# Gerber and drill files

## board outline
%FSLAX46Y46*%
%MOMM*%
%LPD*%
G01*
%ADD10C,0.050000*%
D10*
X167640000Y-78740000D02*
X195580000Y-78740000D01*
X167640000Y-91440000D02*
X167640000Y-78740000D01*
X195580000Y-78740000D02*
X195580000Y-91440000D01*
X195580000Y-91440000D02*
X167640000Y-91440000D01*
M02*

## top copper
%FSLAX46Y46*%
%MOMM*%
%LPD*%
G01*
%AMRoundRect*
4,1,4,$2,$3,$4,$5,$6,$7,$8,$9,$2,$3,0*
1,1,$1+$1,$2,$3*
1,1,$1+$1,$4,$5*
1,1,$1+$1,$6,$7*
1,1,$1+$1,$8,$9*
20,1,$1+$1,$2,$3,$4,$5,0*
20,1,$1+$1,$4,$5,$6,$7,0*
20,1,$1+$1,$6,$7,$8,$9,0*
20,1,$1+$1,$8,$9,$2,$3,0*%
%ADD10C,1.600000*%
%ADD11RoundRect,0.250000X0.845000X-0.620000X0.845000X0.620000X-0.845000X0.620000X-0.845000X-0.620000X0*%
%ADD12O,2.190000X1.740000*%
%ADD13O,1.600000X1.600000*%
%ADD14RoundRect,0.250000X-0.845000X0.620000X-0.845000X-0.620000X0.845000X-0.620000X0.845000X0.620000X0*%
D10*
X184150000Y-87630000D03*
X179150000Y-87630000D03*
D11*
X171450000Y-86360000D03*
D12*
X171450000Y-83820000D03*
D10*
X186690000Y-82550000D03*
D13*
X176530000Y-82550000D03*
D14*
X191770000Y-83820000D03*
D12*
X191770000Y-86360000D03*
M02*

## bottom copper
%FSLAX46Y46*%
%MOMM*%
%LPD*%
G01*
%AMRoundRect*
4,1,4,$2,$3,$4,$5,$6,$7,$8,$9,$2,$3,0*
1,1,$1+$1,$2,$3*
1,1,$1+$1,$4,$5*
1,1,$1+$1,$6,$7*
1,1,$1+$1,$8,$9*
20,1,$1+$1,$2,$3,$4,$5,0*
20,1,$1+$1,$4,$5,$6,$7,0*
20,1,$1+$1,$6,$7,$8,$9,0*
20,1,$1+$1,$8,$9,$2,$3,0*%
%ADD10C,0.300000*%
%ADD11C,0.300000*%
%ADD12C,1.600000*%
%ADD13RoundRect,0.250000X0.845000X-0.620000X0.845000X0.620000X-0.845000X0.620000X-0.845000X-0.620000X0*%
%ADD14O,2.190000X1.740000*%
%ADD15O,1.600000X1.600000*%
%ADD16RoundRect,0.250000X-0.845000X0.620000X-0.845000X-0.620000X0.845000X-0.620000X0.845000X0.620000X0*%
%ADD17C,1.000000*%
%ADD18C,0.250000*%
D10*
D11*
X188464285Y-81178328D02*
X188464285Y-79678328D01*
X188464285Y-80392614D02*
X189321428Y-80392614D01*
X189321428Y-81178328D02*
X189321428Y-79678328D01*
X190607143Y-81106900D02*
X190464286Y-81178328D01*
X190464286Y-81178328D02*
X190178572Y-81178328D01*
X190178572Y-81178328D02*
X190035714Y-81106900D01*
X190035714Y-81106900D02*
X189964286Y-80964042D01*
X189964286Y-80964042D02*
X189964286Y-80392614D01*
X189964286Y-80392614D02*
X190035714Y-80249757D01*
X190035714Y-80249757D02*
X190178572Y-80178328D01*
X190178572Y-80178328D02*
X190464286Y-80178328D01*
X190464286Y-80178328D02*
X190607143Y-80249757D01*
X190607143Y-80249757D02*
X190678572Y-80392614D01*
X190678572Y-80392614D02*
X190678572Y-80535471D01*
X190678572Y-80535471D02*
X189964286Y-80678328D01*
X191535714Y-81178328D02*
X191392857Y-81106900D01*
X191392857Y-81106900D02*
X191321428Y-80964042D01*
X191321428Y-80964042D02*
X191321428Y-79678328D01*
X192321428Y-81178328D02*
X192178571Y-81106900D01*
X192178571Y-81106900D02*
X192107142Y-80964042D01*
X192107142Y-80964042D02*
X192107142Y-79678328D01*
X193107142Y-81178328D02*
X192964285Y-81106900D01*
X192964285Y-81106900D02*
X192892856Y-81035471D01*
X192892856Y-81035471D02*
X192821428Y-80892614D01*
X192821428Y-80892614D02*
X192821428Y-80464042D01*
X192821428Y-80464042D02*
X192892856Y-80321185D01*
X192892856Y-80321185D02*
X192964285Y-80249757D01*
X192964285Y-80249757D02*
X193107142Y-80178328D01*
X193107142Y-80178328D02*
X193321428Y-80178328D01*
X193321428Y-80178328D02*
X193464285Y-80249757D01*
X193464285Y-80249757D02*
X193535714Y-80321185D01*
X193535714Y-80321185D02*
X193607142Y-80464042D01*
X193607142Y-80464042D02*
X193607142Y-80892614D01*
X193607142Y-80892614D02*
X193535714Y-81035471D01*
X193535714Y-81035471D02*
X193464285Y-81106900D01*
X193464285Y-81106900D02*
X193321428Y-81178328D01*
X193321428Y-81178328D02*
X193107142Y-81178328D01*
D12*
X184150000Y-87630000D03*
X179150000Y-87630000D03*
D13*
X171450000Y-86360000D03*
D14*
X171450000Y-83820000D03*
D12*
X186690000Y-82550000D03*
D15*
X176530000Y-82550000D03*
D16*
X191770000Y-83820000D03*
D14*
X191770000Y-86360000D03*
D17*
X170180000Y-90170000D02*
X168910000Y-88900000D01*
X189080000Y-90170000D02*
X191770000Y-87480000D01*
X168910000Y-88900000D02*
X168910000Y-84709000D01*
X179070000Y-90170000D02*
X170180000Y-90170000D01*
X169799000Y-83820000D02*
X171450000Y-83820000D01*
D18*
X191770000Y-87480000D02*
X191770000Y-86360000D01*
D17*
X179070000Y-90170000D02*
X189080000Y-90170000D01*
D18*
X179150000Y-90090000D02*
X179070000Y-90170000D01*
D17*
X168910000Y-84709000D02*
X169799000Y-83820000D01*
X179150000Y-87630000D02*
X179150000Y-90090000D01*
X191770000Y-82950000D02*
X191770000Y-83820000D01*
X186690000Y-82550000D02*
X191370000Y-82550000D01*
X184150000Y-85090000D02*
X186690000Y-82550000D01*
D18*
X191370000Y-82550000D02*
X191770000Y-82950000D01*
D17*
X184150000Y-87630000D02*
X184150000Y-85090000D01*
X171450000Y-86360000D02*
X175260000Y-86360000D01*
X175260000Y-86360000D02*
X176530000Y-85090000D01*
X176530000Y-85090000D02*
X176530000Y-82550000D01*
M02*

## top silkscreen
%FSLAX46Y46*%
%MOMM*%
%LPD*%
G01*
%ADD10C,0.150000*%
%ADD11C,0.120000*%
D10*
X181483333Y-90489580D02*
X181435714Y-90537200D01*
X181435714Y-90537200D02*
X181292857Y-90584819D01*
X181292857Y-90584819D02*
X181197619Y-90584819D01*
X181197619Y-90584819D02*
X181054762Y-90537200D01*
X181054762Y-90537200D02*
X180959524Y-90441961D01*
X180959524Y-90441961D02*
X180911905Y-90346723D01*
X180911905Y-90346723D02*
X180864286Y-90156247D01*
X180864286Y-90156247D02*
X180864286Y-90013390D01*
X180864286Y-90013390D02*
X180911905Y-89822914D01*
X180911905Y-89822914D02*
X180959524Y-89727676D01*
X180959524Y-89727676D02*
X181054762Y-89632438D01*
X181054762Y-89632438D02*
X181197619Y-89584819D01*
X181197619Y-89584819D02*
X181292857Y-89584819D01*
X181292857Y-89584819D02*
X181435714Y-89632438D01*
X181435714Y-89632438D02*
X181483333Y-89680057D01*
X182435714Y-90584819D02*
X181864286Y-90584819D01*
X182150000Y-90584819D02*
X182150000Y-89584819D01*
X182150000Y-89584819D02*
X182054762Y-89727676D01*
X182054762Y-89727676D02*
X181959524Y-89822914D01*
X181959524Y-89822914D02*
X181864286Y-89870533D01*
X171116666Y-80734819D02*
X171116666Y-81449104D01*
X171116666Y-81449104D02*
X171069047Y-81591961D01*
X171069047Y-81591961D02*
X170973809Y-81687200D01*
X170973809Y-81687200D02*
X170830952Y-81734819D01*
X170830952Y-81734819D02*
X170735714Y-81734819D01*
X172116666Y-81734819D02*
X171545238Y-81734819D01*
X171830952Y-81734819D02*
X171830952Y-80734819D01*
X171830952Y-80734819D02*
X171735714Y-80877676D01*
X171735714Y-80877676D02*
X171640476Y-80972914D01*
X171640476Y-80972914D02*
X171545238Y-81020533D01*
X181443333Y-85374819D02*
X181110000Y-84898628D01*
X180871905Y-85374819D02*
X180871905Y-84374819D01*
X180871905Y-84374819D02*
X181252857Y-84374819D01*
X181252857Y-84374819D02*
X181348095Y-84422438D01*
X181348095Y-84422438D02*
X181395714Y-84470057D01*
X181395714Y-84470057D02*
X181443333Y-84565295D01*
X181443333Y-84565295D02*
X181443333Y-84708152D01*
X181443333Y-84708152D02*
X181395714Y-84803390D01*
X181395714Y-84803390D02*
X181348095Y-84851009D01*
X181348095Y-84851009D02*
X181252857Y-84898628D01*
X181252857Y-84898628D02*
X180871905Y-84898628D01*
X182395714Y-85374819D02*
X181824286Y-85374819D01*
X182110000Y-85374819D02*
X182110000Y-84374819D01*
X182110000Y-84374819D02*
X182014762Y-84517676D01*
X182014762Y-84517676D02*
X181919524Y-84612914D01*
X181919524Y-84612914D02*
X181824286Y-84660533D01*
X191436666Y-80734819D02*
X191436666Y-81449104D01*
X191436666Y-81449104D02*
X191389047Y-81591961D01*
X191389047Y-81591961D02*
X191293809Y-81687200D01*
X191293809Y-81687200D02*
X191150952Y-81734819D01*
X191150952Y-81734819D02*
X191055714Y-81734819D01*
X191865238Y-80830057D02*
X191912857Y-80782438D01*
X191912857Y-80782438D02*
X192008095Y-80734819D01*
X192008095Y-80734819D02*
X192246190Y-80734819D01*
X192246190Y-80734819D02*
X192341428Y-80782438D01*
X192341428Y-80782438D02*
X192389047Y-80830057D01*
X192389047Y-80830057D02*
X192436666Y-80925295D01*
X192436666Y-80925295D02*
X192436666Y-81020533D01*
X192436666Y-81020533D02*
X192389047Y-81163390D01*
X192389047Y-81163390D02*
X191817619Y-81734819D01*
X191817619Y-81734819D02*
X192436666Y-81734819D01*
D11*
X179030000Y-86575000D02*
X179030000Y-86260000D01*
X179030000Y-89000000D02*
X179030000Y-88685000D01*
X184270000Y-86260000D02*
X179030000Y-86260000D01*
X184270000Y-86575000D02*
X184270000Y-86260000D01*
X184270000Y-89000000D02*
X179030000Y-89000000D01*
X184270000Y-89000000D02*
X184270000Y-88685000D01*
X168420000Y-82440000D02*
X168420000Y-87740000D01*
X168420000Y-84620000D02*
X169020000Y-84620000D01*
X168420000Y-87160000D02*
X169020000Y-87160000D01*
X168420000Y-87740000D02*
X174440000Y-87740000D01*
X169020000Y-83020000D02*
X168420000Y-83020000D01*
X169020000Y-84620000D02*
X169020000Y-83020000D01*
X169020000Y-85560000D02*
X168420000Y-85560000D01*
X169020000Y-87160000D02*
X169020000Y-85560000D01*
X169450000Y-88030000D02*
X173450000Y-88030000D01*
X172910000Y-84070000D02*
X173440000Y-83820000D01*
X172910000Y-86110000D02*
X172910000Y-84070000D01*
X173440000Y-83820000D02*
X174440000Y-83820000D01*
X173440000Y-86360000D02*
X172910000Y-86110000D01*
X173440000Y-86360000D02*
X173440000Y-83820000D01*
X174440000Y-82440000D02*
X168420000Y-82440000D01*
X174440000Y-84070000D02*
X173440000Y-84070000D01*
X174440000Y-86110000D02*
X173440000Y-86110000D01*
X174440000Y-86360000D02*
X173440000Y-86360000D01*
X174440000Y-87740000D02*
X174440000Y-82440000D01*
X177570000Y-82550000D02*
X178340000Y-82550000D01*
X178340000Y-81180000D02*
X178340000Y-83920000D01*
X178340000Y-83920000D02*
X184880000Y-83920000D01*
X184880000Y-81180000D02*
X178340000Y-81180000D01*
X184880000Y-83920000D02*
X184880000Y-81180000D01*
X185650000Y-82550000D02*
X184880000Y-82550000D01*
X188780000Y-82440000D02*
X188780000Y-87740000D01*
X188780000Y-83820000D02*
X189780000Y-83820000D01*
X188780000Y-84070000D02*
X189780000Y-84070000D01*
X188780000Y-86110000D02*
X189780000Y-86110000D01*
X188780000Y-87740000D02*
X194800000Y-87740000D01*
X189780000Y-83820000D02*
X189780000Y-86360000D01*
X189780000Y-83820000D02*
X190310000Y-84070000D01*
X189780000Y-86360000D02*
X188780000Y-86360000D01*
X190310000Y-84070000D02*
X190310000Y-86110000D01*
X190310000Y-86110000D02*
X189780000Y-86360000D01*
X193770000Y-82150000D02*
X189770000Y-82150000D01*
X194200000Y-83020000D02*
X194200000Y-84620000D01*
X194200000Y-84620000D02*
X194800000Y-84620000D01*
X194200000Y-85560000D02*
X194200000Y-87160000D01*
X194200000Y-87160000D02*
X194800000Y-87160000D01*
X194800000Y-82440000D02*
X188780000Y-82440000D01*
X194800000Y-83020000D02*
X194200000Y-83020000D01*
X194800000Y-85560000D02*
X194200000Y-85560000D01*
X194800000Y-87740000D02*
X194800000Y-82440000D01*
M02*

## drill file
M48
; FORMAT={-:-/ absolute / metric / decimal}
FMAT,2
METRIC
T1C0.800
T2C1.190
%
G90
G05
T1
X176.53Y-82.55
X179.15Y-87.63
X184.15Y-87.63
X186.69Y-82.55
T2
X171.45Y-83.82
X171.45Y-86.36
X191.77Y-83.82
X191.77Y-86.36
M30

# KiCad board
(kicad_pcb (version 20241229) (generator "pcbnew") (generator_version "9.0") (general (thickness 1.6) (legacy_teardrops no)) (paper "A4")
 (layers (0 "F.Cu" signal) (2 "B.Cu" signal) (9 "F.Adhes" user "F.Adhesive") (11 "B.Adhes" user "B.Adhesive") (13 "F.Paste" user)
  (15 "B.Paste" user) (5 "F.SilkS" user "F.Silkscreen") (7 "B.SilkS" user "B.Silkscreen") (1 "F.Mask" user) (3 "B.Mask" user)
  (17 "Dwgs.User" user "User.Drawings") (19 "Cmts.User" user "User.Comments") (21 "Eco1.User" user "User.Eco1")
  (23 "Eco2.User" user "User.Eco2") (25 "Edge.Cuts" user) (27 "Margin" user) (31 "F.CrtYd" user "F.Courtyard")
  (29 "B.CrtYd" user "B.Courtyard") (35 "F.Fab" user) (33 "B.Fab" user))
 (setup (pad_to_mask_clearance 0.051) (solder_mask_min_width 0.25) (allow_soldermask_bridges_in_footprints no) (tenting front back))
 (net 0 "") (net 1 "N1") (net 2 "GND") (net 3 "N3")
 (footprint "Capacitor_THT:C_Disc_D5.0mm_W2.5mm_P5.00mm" (layer "F.Cu") (at 184.15 87.63 180)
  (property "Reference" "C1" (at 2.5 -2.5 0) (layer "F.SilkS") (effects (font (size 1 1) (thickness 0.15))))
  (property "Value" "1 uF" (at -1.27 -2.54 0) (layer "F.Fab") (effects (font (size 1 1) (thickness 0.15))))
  (fp_line (start 5.12 1.055) (end 5.12 1.37) (stroke (width 0.12) (type solid)) (layer "F.SilkS"))
  (fp_line (start 5.12 -1.37) (end 5.12 -1.055) (stroke (width 0.12) (type solid)) (layer "F.SilkS"))
  (fp_line (start -0.12 1.37) (end 5.12 1.37) (stroke (width 0.12) (type solid)) (layer "F.SilkS"))
  (fp_line (start -0.12 1.055) (end -0.12 1.37) (stroke (width 0.12) (type solid)) (layer "F.SilkS"))
  (fp_line (start -0.12 -1.37) (end 5.12 -1.37) (stroke (width 0.12) (type solid)) (layer "F.SilkS"))
  (fp_line (start -0.12 -1.37) (end -0.12 -1.055) (stroke (width 0.12) (type solid)) (layer "F.SilkS"))
  (pad "1" thru_hole circle (at 0 0 180) (size 1.6 1.6) (drill 0.8) (layers "*.Cu" "*.Mask") (remove_unused_layers no) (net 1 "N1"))
  (pad "2" thru_hole circle (at 5 0 180) (size 1.6 1.6) (drill 0.8) (layers "*.Cu" "*.Mask") (remove_unused_layers no) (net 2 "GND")))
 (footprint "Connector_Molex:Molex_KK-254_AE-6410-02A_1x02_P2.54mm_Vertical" (layer "F.Cu") (at 171.45 86.36 90)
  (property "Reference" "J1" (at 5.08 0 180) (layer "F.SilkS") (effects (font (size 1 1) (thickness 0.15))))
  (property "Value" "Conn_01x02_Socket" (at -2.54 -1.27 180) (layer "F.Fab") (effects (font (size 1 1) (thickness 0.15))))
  (fp_line (start 3.92 -3.03) (end -1.38 -3.03) (stroke (width 0.12) (type solid)) (layer "F.SilkS"))
  (fp_line (start 1.74 -3.03) (end 1.74 -2.43) (stroke (width 0.12) (type solid)) (layer "F.SilkS"))
  (fp_line (start -0.8 -3.03) (end -0.8 -2.43) (stroke (width 0.12) (type solid)) (layer "F.SilkS"))
  (fp_line (start -1.38 -3.03) (end -1.38 2.99) (stroke (width 0.12) (type solid)) (layer "F.SilkS"))
  (fp_line (start 3.34 -2.43) (end 3.34 -3.03) (stroke (width 0.12) (type solid)) (layer "F.SilkS"))
  (fp_line (start 1.74 -2.43) (end 3.34 -2.43) (stroke (width 0.12) (type solid)) (layer "F.SilkS"))
  (fp_line (start 0.8 -2.43) (end 0.8 -3.03) (stroke (width 0.12) (type solid)) (layer "F.SilkS"))
  (fp_line (start -0.8 -2.43) (end 0.8 -2.43) (stroke (width 0.12) (type solid)) (layer "F.SilkS"))
  (fp_line (start -1.67 -2) (end -1.67 2) (stroke (width 0.12) (type solid)) (layer "F.SilkS"))
  (fp_line (start 2.29 1.46) (end 2.54 1.99) (stroke (width 0.12) (type solid)) (layer "F.SilkS"))
  (fp_line (start 0.25 1.46) (end 2.29 1.46) (stroke (width 0.12) (type solid)) (layer "F.SilkS"))
  (fp_line (start 2.54 1.99) (end 2.54 2.99) (stroke (width 0.12) (type solid)) (layer "F.SilkS"))
  (fp_line (start 0 1.99) (end 0.25 1.46) (stroke (width 0.12) (type solid)) (layer "F.SilkS"))
  (fp_line (start 0 1.99) (end 2.54 1.99) (stroke (width 0.12) (type solid)) (layer "F.SilkS"))
  (fp_line (start 3.92 2.99) (end 3.92 -3.03) (stroke (width 0.12) (type solid)) (layer "F.SilkS"))
  (fp_line (start 2.29 2.99) (end 2.29 1.99) (stroke (width 0.12) (type solid)) (layer "F.SilkS"))
  (fp_line (start 0.25 2.99) (end 0.25 1.99) (stroke (width 0.12) (type solid)) (layer "F.SilkS"))
  (fp_line (start 0 2.99) (end 0 1.99) (stroke (width 0.12) (type solid)) (layer "F.SilkS"))
  (fp_line (start -1.38 2.99) (end 3.92 2.99) (stroke (width 0.12) (type solid)) (layer "F.SilkS"))
  (pad "1" thru_hole roundrect (at 0 0 90) (size 1.74 2.19) (drill 1.19) (layers "*.Cu" "*.Mask") (remove_unused_layers no)
   (roundrect_rratio 0.143678) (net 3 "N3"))
  (pad "2" thru_hole oval (at 2.54 0 90) (size 1.74 2.19) (drill 1.19) (layers "*.Cu" "*.Mask") (remove_unused_layers no) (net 2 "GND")))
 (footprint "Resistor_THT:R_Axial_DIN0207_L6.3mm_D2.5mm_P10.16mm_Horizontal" (layer "F.Cu") (at 186.69 82.55 180)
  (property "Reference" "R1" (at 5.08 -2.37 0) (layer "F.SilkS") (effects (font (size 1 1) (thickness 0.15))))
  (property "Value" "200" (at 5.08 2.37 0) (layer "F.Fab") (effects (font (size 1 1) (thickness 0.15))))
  (fp_line (start 9.12 0) (end 8.35 0) (stroke (width 0.12) (type solid)) (layer "F.SilkS"))
  (fp_line (start 8.35 1.37) (end 8.35 -1.37) (stroke (width 0.12) (type solid)) (layer "F.SilkS"))
  (fp_line (start 8.35 -1.37) (end 1.81 -1.37) (stroke (width 0.12) (type solid)) (layer "F.SilkS"))
  (fp_line (start 1.81 1.37) (end 8.35 1.37) (stroke (width 0.12) (type solid)) (layer "F.SilkS"))
  (fp_line (start 1.81 -1.37) (end 1.81 1.37) (stroke (width 0.12) (type solid)) (layer "F.SilkS"))
  (fp_line (start 1.04 0) (end 1.81 0) (stroke (width 0.12) (type solid)) (layer "F.SilkS"))
  (pad "1" thru_hole circle (at 0 0 180) (size 1.6 1.6) (drill 0.8) (layers "*.Cu" "*.Mask") (remove_unused_layers no) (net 1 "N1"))
  (pad "2" thru_hole oval (at 10.16 0 180) (size 1.6 1.6) (drill 0.8) (layers "*.Cu" "*.Mask") (remove_unused_layers no) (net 3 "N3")))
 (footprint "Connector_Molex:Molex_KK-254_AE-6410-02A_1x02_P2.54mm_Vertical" (layer "F.Cu") (at 191.77 83.82 -90)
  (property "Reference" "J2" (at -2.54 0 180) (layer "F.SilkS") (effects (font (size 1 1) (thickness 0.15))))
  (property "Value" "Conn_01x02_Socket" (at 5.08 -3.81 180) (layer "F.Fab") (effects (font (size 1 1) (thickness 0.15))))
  (fp_line (start -1.38 2.99) (end 3.92 2.99) (stroke (width 0.12) (type solid)) (layer "F.SilkS"))
  (fp_line (start 0 2.99) (end 0 1.99) (stroke (width 0.12) (type solid)) (layer "F.SilkS"))
  (fp_line (start 0.25 2.99) (end 0.25 1.99) (stroke (width 0.12) (type solid)) (layer "F.SilkS"))
  (fp_line (start 2.29 2.99) (end 2.29 1.99) (stroke (width 0.12) (type solid)) (layer "F.SilkS"))
  (fp_line (start 3.92 2.99) (end 3.92 -3.03) (stroke (width 0.12) (type solid)) (layer "F.SilkS"))
  (fp_line (start 0 1.99) (end 2.54 1.99) (stroke (width 0.12) (type solid)) (layer "F.SilkS"))
  (fp_line (start 0 1.99) (end 0.25 1.46) (stroke (width 0.12) (type solid)) (layer "F.SilkS"))
  (fp_line (start 2.54 1.99) (end 2.54 2.99) (stroke (width 0.12) (type solid)) (layer "F.SilkS"))
  (fp_line (start 0.25 1.46) (end 2.29 1.46) (stroke (width 0.12) (type solid)) (layer "F.SilkS"))
  (fp_line (start 2.29 1.46) (end 2.54 1.99) (stroke (width 0.12) (type solid)) (layer "F.SilkS"))
  (fp_line (start -1.67 -2) (end -1.67 2) (stroke (width 0.12) (type solid)) (layer "F.SilkS"))
  (fp_line (start -0.8 -2.43) (end 0.8 -2.43) (stroke (width 0.12) (type solid)) (layer "F.SilkS"))
  (fp_line (start 0.8 -2.43) (end 0.8 -3.03) (stroke (width 0.12) (type solid)) (layer "F.SilkS"))
  (fp_line (start 1.74 -2.43) (end 3.34 -2.43) (stroke (width 0.12) (type solid)) (layer "F.SilkS"))
  (fp_line (start 3.34 -2.43) (end 3.34 -3.03) (stroke (width 0.12) (type solid)) (layer "F.SilkS"))
  (fp_line (start -1.38 -3.03) (end -1.38 2.99) (stroke (width 0.12) (type solid)) (layer "F.SilkS"))
  (fp_line (start -0.8 -3.03) (end -0.8 -2.43) (stroke (width 0.12) (type solid)) (layer "F.SilkS"))
  (fp_line (start 1.74 -3.03) (end 1.74 -2.43) (stroke (width 0.12) (type solid)) (layer "F.SilkS"))
  (fp_line (start 3.92 -3.03) (end -1.38 -3.03) (stroke (width 0.12) (type solid)) (layer "F.SilkS"))
  (pad "1" thru_hole roundrect (at 0 0 270) (size 1.74 2.19) (drill 1.19) (layers "*.Cu" "*.Mask") (remove_unused_layers no)
   (roundrect_rratio 0.143678) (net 1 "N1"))
  (pad "2" thru_hole oval (at 2.54 0 270) (size 1.74 2.19) (drill 1.19) (layers "*.Cu" "*.Mask") (remove_unused_layers no) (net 2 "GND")))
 (gr_line (start 167.64 78.74) (end 195.58 78.74) (stroke (width 0.05) (type solid)) (layer "Edge.Cuts"))
 (gr_line (start 167.64 91.44) (end 167.64 78.74) (stroke (width 0.05) (type solid)) (layer "Edge.Cuts"))
 (gr_line (start 195.58 78.74) (end 195.58 91.44) (stroke (width 0.05) (type solid)) (layer "Edge.Cuts"))
 (gr_line (start 195.58 91.44) (end 167.64 91.44) (stroke (width 0.05) (type solid)) (layer "Edge.Cuts"))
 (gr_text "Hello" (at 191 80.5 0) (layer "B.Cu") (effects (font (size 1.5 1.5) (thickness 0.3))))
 (segment (start 170.18 90.17) (end 168.91 88.9) (width 1) (layer "B.Cu") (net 2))
 (segment (start 189.08 90.17) (end 191.77 87.48) (width 1) (layer "B.Cu") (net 2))
 (segment (start 168.91 88.9) (end 168.91 84.709) (width 1) (layer "B.Cu") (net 2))
 (segment (start 179.07 90.17) (end 170.18 90.17) (width 1) (layer "B.Cu") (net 2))
 (segment (start 169.799 83.82) (end 171.45 83.82) (width 1) (layer "B.Cu") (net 2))
 (segment (start 191.77 87.48) (end 191.77 86.36) (width 0.25) (layer "B.Cu") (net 2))
 (segment (start 179.07 90.17) (end 189.08 90.17) (width 1) (layer "B.Cu") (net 2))
 (segment (start 179.15 90.09) (end 179.07 90.17) (width 0.25) (layer "B.Cu") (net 2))
 (segment (start 168.91 84.709) (end 169.799 83.82) (width 1) (layer "B.Cu") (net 2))
 (segment (start 179.15 87.63) (end 179.15 90.09) (width 1) (layer "B.Cu") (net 2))
 (segment (start 191.77 82.95) (end 191.77 83.82) (width 1) (layer "B.Cu") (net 1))
 (segment (start 186.69 82.55) (end 191.37 82.55) (width 1) (layer "B.Cu") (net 1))
 (segment (start 184.15 85.09) (end 186.69 82.55) (width 1) (layer "B.Cu") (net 1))
 (segment (start 191.37 82.55) (end 191.77 82.95) (width 0.25) (layer "B.Cu") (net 1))
 (segment (start 184.15 87.63) (end 184.15 85.09) (width 1) (layer "B.Cu") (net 1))
 (segment (start 171.45 86.36) (end 175.26 86.36) (width 1) (layer "B.Cu") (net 3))
 (segment (start 175.26 86.36) (end 176.53 85.09) (width 1) (layer "B.Cu") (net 3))
 (segment (start 176.53 85.09) (end 176.53 82.55) (width 1) (layer "B.Cu") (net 3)))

